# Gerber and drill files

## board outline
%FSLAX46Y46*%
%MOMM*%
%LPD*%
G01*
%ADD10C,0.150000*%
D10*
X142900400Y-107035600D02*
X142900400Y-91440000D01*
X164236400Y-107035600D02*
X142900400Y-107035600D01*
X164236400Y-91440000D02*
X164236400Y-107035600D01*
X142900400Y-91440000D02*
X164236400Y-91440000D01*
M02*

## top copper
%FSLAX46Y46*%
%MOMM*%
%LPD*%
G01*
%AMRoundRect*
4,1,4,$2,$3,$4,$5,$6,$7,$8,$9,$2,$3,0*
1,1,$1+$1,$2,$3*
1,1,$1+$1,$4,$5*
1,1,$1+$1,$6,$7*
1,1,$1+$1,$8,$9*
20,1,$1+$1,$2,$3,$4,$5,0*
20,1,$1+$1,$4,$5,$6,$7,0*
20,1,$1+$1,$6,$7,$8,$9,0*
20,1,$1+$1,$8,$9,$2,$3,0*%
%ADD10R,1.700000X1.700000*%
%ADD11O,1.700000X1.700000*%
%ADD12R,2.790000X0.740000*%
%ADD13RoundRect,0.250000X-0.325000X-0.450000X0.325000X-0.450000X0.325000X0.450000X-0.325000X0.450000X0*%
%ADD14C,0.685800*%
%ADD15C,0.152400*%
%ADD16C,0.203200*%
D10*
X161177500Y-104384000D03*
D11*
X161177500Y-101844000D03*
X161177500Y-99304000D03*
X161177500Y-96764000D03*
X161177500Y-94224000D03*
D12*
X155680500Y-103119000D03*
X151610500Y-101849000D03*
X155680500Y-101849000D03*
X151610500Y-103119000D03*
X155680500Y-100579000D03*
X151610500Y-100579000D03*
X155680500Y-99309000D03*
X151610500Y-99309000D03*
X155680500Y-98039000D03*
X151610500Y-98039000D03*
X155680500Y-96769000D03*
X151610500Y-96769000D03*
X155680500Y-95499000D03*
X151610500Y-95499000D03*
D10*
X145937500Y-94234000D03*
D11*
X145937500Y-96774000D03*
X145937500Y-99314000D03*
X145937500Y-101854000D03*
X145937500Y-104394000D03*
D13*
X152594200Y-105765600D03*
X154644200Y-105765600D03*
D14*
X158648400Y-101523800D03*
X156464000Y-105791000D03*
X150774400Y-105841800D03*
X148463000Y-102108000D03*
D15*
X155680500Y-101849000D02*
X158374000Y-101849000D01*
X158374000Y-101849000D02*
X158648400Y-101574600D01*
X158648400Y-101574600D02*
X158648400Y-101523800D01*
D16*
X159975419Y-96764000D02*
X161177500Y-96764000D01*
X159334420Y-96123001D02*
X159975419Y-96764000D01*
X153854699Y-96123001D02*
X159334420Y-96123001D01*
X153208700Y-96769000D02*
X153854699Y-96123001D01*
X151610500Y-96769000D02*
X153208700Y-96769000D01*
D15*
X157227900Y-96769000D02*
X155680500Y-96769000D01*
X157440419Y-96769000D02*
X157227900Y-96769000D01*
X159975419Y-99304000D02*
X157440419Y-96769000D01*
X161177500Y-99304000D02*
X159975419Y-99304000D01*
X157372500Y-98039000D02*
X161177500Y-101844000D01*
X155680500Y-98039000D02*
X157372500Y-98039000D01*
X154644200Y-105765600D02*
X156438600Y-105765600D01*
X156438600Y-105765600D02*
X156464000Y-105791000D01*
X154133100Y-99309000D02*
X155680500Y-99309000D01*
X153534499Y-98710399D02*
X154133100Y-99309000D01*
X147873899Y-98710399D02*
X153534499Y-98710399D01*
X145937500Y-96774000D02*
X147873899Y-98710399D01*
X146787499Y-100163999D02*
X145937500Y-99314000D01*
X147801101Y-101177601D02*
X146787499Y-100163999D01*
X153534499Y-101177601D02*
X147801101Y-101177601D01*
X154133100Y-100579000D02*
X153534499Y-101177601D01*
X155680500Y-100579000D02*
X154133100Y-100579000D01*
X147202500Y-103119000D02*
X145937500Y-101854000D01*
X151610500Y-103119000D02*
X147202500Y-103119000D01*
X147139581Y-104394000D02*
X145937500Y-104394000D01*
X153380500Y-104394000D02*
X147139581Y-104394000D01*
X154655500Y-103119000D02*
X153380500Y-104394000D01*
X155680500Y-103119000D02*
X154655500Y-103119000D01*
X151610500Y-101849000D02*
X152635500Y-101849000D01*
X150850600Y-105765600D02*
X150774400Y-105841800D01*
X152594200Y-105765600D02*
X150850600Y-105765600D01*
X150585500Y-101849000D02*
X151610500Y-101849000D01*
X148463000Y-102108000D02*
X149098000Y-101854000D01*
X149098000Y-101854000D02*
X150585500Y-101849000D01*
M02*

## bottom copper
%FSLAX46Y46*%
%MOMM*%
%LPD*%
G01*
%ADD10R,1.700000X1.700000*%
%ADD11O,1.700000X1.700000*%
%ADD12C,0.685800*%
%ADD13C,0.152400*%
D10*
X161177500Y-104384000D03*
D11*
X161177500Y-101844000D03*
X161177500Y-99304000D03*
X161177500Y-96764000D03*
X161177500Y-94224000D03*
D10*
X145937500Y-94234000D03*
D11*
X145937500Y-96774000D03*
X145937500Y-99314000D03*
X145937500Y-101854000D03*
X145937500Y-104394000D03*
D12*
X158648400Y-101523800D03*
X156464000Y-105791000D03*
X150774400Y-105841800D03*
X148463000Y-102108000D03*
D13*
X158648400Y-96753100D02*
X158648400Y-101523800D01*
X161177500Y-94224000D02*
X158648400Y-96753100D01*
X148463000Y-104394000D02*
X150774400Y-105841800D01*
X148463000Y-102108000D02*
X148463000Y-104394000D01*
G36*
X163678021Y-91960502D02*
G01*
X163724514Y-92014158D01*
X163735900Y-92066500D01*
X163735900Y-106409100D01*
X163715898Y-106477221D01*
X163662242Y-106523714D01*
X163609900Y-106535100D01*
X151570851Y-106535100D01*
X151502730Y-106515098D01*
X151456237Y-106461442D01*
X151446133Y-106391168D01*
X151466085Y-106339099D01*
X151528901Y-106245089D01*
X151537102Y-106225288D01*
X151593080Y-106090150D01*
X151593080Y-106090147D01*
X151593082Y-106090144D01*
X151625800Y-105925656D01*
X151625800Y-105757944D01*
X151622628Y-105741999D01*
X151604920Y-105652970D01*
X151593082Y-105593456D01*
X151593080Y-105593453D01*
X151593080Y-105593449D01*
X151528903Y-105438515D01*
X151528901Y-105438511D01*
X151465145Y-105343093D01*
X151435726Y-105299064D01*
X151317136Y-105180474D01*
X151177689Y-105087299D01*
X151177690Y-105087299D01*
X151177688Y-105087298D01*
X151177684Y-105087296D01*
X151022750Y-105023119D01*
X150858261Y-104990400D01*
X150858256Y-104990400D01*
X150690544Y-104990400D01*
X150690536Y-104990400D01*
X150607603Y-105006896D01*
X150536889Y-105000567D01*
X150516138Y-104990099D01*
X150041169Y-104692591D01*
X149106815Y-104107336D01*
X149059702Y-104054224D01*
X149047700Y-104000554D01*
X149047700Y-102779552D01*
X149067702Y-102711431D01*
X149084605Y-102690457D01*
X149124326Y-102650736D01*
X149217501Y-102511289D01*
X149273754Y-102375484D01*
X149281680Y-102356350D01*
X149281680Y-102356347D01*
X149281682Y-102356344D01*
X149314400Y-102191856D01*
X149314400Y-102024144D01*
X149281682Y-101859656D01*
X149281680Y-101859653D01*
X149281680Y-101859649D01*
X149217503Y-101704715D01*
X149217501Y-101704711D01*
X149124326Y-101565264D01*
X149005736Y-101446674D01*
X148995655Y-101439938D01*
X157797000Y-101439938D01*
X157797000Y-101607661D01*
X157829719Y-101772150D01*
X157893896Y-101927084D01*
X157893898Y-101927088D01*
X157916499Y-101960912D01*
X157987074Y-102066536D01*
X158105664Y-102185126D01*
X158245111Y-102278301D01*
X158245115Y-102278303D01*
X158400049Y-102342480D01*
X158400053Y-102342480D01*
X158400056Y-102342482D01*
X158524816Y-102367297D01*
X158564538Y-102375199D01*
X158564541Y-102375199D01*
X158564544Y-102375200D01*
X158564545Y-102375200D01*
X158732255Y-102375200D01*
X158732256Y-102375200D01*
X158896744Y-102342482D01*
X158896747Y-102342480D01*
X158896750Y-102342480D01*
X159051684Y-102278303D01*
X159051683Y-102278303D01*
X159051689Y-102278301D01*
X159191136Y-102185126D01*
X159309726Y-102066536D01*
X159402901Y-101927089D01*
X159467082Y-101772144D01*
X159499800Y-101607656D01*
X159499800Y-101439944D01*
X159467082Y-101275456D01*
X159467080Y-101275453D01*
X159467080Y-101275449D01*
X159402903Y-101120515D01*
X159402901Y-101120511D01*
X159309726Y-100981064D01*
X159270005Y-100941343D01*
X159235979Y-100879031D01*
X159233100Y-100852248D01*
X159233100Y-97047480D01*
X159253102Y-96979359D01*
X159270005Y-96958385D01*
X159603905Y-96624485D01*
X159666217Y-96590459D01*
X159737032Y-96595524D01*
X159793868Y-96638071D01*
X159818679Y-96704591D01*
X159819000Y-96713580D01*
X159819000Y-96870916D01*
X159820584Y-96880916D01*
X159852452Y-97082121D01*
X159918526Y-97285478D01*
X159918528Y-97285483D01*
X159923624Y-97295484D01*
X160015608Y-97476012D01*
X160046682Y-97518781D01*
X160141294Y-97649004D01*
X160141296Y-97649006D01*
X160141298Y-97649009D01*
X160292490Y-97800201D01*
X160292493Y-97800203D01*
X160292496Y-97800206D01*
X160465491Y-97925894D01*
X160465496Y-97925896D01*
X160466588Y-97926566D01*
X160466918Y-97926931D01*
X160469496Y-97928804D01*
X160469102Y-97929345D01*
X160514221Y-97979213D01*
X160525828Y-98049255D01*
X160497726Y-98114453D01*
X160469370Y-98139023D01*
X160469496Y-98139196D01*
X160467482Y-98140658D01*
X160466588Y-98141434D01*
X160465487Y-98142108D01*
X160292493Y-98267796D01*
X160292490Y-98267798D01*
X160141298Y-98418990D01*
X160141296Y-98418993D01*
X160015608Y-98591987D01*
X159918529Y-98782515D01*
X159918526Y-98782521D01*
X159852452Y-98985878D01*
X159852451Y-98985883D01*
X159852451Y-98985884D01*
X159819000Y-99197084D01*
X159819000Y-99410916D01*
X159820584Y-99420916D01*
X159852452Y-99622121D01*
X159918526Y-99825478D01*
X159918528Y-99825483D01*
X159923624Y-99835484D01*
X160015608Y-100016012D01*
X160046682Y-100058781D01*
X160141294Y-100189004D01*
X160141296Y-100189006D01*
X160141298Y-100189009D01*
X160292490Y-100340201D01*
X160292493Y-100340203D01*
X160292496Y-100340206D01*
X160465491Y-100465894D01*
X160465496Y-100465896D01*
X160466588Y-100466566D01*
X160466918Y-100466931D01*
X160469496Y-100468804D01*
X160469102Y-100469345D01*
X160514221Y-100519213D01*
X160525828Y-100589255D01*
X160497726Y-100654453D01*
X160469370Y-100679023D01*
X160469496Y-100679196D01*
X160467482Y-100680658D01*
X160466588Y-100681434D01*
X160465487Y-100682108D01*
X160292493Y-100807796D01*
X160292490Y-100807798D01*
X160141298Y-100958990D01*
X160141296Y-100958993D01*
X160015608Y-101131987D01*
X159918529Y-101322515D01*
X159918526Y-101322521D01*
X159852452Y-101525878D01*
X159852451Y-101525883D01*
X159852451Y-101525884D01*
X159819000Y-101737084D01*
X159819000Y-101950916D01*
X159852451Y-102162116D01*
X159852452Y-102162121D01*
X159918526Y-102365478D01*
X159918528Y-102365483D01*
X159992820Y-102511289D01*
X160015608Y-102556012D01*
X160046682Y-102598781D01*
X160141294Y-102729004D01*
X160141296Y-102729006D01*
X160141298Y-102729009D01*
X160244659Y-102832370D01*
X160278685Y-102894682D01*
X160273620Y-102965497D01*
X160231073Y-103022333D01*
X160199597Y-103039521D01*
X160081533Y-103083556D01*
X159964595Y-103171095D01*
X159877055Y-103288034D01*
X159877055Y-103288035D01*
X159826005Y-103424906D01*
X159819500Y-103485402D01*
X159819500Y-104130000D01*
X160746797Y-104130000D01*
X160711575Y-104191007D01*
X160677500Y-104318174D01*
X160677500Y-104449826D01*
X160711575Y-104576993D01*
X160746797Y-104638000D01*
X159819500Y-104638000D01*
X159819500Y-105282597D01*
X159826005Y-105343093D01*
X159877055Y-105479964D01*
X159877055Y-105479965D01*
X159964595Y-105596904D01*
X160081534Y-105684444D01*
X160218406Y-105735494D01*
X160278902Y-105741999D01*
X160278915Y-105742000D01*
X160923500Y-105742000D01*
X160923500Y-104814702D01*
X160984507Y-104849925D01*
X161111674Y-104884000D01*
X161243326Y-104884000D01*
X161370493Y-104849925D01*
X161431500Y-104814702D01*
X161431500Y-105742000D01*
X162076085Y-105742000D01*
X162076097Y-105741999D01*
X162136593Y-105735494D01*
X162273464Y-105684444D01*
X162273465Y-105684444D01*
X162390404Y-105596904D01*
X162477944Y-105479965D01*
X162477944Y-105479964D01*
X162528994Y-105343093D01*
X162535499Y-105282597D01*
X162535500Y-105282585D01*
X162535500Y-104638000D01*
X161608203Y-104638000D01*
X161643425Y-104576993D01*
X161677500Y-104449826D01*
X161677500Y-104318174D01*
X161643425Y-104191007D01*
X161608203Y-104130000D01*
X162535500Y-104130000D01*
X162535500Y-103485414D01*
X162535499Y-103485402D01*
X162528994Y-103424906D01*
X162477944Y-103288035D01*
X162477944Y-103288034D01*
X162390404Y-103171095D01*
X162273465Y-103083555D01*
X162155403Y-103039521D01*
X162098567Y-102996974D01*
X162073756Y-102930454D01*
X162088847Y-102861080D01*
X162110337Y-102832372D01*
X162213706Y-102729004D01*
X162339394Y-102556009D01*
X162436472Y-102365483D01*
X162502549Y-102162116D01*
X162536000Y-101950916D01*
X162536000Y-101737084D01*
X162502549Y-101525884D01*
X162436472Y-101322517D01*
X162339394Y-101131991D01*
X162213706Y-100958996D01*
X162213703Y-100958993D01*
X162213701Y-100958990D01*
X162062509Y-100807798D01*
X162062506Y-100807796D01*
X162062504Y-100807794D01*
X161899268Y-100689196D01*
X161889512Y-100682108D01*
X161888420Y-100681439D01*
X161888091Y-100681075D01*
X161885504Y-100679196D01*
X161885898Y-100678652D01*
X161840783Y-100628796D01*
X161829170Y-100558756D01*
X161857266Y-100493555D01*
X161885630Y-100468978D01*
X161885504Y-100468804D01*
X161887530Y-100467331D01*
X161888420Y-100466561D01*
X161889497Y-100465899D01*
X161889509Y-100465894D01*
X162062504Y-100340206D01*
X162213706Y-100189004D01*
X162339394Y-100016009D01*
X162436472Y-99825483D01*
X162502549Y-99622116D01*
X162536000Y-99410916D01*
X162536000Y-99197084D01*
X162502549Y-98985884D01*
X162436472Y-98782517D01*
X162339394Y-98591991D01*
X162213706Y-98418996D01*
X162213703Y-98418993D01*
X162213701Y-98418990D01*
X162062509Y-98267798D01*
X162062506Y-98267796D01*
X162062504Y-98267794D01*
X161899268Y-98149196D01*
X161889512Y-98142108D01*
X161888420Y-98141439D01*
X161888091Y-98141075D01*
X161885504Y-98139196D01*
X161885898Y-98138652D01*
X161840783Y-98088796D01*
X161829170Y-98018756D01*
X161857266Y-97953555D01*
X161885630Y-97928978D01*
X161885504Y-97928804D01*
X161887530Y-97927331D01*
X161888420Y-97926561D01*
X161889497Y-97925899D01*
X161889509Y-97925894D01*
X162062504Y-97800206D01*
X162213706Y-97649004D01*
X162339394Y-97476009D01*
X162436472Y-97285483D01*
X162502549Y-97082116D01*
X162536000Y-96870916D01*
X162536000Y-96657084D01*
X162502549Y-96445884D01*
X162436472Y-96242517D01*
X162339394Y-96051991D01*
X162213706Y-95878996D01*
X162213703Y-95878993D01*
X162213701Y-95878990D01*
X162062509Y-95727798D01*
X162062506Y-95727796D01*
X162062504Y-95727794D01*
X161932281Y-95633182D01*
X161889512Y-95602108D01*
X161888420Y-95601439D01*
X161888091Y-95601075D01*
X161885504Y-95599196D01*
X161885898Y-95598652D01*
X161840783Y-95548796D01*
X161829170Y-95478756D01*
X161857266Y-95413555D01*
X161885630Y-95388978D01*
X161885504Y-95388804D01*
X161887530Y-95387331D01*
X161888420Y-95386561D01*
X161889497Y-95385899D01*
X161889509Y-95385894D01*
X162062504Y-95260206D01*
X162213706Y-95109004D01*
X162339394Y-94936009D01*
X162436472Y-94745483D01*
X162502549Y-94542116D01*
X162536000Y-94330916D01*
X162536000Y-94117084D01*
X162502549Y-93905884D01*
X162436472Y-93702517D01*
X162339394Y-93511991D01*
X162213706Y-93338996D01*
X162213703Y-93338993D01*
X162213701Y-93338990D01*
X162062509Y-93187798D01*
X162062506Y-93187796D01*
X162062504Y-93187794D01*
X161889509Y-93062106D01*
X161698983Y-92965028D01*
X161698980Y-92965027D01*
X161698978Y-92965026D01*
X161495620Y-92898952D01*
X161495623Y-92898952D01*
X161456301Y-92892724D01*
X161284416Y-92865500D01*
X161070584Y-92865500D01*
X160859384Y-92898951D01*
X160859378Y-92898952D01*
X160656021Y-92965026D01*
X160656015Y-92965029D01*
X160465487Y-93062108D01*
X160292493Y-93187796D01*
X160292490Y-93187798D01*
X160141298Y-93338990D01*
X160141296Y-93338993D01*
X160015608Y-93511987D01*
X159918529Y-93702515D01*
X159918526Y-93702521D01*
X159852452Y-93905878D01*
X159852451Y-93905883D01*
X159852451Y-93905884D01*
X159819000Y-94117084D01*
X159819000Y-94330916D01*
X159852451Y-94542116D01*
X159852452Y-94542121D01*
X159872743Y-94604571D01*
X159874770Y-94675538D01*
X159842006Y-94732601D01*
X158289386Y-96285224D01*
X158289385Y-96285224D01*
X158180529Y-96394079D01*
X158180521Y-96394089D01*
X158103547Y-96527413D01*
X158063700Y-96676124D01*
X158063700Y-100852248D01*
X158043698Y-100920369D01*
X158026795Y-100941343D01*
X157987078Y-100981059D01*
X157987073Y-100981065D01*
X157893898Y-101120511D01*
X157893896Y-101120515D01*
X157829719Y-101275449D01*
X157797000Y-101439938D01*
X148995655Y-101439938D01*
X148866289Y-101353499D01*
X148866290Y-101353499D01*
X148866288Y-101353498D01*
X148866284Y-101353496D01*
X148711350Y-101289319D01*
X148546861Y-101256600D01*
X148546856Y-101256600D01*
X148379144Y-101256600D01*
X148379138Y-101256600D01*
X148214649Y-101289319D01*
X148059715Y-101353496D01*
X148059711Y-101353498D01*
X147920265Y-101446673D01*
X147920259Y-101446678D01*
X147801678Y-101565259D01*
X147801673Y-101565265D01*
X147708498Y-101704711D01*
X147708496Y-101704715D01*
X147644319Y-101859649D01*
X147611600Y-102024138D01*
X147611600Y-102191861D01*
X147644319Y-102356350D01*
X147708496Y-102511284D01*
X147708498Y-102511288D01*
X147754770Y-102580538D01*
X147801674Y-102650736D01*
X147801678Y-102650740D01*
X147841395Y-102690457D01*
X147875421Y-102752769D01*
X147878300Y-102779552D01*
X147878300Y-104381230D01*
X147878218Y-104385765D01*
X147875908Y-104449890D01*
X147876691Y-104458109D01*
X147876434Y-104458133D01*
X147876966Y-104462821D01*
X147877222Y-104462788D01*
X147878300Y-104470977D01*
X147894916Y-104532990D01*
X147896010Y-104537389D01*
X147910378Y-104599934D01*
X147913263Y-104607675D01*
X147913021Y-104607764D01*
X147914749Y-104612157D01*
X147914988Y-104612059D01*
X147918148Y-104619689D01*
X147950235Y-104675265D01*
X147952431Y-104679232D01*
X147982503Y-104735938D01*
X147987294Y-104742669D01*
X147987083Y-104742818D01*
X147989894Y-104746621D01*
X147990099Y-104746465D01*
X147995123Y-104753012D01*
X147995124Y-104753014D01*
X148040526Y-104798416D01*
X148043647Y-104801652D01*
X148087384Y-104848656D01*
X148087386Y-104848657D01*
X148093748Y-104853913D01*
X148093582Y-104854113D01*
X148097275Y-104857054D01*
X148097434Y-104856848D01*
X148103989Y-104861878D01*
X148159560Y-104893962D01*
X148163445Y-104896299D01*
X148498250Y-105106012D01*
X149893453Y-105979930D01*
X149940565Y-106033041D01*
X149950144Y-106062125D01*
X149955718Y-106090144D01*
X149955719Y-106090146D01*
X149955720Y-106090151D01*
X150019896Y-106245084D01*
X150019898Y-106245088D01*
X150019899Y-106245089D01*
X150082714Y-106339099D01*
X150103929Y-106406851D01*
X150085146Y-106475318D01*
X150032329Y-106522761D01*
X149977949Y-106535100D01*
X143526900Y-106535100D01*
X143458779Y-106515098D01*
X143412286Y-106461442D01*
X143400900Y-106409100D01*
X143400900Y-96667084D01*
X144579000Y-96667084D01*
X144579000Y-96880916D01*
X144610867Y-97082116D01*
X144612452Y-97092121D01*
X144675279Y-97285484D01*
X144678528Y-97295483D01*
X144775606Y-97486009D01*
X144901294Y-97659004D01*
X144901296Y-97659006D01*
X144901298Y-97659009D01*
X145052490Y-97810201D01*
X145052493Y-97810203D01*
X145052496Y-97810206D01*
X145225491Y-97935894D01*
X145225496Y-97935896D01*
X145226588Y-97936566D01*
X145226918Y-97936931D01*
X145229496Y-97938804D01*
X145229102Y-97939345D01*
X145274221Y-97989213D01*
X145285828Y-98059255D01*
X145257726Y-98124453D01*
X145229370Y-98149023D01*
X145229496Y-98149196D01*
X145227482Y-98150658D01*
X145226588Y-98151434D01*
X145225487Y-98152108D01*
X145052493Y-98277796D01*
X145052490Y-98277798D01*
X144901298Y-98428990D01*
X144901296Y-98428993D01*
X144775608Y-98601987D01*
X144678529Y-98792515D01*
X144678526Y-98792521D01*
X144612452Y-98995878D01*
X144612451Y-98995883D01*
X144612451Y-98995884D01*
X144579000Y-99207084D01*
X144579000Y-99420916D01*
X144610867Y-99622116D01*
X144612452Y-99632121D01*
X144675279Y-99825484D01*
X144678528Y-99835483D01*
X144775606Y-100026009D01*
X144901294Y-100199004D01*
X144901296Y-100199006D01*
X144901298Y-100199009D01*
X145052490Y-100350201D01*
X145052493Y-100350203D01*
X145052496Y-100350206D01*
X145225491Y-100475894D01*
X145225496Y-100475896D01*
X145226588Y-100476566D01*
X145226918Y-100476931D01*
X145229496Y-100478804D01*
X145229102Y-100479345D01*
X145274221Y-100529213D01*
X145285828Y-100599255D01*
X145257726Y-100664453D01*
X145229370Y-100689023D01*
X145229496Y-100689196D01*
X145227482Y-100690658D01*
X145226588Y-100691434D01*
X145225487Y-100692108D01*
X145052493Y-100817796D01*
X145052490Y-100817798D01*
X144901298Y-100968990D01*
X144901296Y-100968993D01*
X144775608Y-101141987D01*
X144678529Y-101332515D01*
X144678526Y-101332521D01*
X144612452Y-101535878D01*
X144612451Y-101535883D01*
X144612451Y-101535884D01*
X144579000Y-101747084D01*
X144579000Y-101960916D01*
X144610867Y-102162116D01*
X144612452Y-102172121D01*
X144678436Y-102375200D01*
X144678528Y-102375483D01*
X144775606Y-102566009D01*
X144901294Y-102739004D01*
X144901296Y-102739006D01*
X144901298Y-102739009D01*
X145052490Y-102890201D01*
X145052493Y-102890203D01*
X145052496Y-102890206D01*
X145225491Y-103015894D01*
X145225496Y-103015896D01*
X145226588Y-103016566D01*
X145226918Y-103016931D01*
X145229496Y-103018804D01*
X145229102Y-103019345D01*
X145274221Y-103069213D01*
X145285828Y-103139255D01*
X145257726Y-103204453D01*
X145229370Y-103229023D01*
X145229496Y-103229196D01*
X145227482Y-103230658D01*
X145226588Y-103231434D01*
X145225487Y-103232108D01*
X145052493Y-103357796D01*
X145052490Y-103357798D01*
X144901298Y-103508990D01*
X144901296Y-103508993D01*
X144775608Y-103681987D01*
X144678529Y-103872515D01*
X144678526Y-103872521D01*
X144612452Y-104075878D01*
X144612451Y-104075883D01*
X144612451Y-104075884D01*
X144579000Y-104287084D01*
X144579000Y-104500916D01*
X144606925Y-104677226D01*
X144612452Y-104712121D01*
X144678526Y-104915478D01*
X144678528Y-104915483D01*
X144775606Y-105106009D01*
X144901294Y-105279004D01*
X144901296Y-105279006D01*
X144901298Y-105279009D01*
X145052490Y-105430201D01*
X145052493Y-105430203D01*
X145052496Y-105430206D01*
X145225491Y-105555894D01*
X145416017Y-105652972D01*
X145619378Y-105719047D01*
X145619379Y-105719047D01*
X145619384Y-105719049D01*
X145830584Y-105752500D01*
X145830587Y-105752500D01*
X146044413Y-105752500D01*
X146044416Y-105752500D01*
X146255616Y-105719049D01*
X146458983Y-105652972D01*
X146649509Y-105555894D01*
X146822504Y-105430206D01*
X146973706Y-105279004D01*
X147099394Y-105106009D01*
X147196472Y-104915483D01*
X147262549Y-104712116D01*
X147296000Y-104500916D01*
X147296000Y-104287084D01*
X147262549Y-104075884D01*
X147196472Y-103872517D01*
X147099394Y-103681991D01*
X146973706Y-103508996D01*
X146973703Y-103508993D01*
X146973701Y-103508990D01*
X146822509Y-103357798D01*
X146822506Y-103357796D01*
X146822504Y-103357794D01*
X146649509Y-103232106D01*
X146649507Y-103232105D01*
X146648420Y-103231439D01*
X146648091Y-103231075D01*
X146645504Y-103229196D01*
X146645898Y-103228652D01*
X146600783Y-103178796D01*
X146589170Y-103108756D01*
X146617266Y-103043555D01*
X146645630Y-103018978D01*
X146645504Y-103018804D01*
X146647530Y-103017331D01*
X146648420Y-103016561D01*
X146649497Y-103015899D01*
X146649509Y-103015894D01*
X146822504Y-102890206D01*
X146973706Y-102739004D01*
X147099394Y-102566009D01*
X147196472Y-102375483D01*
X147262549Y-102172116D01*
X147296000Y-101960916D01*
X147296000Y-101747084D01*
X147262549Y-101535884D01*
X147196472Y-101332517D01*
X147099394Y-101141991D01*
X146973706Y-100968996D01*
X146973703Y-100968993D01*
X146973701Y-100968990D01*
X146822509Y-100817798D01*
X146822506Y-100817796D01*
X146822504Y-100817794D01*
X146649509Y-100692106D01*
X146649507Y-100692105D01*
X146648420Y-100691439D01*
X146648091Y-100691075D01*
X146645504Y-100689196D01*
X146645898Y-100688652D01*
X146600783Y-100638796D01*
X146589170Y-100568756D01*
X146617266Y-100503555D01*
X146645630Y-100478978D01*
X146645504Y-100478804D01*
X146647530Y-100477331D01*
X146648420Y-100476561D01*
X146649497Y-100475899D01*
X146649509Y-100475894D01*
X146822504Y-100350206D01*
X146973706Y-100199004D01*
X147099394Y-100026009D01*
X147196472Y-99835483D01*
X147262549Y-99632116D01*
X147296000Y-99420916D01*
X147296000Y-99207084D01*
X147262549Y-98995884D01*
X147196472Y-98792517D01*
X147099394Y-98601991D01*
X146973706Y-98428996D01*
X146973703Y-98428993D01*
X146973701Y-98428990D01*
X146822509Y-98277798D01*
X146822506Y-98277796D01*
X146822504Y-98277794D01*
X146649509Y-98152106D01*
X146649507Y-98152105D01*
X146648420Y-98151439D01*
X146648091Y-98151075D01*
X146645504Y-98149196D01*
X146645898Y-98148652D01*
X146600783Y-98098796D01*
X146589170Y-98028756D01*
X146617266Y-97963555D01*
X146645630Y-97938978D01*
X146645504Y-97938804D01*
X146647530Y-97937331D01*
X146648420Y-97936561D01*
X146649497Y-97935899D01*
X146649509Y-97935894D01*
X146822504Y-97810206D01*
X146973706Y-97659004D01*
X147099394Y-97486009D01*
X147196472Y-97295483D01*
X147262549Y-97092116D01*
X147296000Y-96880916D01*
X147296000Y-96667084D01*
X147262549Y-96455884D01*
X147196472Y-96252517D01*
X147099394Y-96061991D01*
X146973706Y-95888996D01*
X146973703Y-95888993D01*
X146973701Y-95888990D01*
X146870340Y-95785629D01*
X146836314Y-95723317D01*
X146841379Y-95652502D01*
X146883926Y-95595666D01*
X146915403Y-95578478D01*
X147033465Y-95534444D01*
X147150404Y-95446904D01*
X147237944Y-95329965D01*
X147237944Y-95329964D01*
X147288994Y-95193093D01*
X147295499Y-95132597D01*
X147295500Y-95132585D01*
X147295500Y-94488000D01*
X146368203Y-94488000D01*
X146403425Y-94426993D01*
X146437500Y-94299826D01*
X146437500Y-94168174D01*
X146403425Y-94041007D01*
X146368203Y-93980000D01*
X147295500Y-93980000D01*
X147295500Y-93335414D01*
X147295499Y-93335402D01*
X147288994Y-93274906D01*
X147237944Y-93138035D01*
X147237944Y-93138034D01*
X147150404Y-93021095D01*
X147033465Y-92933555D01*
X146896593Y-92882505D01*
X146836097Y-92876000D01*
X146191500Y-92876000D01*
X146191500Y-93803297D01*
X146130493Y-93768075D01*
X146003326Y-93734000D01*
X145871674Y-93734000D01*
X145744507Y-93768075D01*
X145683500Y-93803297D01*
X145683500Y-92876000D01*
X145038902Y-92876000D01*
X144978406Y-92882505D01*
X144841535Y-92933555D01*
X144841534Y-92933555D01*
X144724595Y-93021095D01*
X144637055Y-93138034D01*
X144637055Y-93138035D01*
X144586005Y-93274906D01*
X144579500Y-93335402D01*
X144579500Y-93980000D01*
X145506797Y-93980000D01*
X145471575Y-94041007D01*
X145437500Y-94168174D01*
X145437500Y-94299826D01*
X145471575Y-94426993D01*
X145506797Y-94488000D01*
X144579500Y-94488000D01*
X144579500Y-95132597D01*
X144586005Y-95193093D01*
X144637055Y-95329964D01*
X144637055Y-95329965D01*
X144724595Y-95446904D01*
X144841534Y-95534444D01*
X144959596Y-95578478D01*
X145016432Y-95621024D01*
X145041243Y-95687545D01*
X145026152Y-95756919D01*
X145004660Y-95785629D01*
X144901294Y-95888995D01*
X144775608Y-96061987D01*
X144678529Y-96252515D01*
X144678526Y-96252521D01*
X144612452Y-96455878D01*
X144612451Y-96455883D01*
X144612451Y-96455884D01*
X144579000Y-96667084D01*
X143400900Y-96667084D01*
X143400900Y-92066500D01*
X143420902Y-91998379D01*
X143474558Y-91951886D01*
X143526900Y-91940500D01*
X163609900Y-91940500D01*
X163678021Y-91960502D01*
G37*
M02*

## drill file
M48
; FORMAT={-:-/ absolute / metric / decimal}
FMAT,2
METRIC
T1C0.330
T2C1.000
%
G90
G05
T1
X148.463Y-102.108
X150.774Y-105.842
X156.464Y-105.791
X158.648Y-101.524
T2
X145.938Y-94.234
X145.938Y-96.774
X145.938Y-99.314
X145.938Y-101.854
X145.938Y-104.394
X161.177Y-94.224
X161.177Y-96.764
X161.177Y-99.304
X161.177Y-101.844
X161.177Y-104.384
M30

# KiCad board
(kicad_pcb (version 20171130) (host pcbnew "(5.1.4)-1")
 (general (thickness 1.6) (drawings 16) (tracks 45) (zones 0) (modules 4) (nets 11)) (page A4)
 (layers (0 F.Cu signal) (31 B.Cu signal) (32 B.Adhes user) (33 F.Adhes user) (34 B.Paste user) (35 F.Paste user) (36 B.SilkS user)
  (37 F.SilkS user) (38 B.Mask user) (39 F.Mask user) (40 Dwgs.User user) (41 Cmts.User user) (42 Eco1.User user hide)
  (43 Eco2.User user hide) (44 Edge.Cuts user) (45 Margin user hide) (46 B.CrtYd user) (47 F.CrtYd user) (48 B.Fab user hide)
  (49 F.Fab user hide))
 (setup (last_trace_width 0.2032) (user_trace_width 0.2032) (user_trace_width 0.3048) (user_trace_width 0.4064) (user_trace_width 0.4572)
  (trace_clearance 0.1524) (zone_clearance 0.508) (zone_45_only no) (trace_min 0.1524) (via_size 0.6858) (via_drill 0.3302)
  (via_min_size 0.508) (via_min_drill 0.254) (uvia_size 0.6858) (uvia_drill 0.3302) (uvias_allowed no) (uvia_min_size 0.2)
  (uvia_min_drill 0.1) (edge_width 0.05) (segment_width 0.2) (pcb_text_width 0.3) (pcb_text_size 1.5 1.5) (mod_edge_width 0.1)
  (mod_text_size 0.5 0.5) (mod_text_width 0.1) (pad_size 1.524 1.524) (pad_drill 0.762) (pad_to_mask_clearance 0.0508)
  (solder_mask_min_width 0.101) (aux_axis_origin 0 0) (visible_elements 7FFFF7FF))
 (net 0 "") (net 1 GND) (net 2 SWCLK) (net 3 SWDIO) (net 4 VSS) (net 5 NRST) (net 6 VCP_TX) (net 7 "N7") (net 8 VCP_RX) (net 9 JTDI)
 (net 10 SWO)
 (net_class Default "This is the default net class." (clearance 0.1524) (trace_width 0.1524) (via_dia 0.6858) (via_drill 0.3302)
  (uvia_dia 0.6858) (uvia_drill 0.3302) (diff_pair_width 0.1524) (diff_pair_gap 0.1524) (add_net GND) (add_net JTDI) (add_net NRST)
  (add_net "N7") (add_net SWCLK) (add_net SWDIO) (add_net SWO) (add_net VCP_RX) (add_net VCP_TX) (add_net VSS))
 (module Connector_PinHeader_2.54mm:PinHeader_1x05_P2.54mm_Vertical (layer F.Cu) (at 161.1775 104.384 180)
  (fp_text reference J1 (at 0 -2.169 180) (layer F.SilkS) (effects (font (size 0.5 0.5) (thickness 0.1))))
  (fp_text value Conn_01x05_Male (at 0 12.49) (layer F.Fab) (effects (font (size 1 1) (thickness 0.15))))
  (pad 1 thru_hole rect (at 0 0 180) (size 1.7 1.7) (drill 1) (layers *.Cu *.Mask) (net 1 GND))
  (pad 2 thru_hole oval (at 0 2.54 180) (size 1.7 1.7) (drill 1) (layers *.Cu *.Mask) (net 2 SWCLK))
  (pad 3 thru_hole oval (at 0 5.08 180) (size 1.7 1.7) (drill 1) (layers *.Cu *.Mask) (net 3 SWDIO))
  (pad 4 thru_hole oval (at 0 7.62 180) (size 1.7 1.7) (drill 1) (layers *.Cu *.Mask) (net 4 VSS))
  (pad 5 thru_hole oval (at 0 10.16 180) (size 1.7 1.7) (drill 1) (layers *.Cu *.Mask) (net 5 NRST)))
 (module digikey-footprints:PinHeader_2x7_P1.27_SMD (layer F.Cu) (at 153.6455 99.309 270)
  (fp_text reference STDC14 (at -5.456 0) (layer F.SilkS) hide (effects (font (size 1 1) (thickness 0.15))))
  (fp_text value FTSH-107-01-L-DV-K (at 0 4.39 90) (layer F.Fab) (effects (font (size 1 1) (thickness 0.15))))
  (pad 14 smd rect (at 3.81 -2.035 270) (size 0.74 2.79) (layers F.Cu F.Paste F.Mask) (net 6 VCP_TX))
  (pad 11 smd rect (at 2.54 2.035 270) (size 0.74 2.79) (layers F.Cu F.Paste F.Mask) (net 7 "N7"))
  (pad 12 smd rect (at 2.54 -2.035 270) (size 0.74 2.79) (layers F.Cu F.Paste F.Mask) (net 5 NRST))
  (pad 13 smd rect (at 3.81 2.035 270) (size 0.74 2.79) (layers F.Cu F.Paste F.Mask) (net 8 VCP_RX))
  (pad 10 smd rect (at 1.27 -2.035 270) (size 0.74 2.79) (layers F.Cu F.Paste F.Mask) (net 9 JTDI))
  (pad 9 smd rect (at 1.27 2.035 270) (size 0.74 2.79) (layers F.Cu F.Paste F.Mask))
  (pad 8 smd rect (at 0 -2.035 270) (size 0.74 2.79) (layers F.Cu F.Paste F.Mask) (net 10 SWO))
  (pad 7 smd rect (at 0 2.035 270) (size 0.74 2.79) (layers F.Cu F.Paste F.Mask) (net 1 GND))
  (pad 6 smd rect (at -1.27 -2.035 270) (size 0.74 2.79) (layers F.Cu F.Paste F.Mask) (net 2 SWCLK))
  (pad 5 smd rect (at -1.27 2.035 270) (size 0.74 2.79) (layers F.Cu F.Paste F.Mask) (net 1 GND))
  (pad 4 smd rect (at -2.54 -2.035 270) (size 0.74 2.79) (layers F.Cu F.Paste F.Mask) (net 3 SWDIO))
  (pad 3 smd rect (at -2.54 2.035 270) (size 0.74 2.79) (layers F.Cu F.Paste F.Mask) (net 4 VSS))
  (pad 2 smd rect (at -3.81 -2.035 270) (size 0.74 2.79) (layers F.Cu F.Paste F.Mask))
  (pad 1 smd rect (at -3.81 2.035 270) (size 0.74 2.79) (layers F.Cu F.Paste F.Mask)))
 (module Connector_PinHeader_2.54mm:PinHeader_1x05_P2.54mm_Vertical (layer F.Cu) (at 145.9375 94.234)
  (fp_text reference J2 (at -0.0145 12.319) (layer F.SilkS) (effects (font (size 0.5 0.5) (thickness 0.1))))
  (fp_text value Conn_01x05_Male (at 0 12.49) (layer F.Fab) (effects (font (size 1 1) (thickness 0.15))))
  (pad 1 thru_hole rect (at 0 0) (size 1.7 1.7) (drill 1) (layers *.Cu *.Mask) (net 1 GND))
  (pad 2 thru_hole oval (at 0 2.54) (size 1.7 1.7) (drill 1) (layers *.Cu *.Mask) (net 10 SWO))
  (pad 3 thru_hole oval (at 0 5.08) (size 1.7 1.7) (drill 1) (layers *.Cu *.Mask) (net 9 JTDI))
  (pad 4 thru_hole oval (at 0 7.62) (size 1.7 1.7) (drill 1) (layers *.Cu *.Mask) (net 8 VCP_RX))
  (pad 5 thru_hole oval (at 0 10.16) (size 1.7 1.7) (drill 1) (layers *.Cu *.Mask) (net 6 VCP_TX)))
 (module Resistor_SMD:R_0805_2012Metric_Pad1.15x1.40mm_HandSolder (layer F.Cu) (at 153.6192 105.7656)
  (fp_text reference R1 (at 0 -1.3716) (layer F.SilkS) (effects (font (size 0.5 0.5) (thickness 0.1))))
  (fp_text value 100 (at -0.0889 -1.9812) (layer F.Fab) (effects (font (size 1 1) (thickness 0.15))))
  (pad 1 smd roundrect (at -1.025 0) (size 1.15 1.4) (layers F.Cu F.Paste F.Mask) (roundrect_rratio 0.217391) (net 7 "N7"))
  (pad 2 smd roundrect (at 1.025 0) (size 1.15 1.4) (layers F.Cu F.Paste F.Mask) (roundrect_rratio 0.217391) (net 1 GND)))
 (gr_line (start 142.9004 107.0356) (end 142.9004 91.44) (layer Edge.Cuts) (width 0.15))
 (gr_line (start 164.2364 107.0356) (end 142.9004 107.0356) (layer Edge.Cuts) (width 0.15))
 (gr_line (start 164.2364 91.44) (end 164.2364 107.0356) (layer Edge.Cuts) (width 0.15))
 (gr_line (start 142.9004 91.44) (end 164.2364 91.44) (layer Edge.Cuts) (width 0.15))
 (segment (start 155.6805 101.849) (end 158.374 101.849) (width 0.1524) (layer F.Cu) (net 5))
 (via (at 158.6484 101.5238) (size 0.6858) (drill 0.3302) (layers F.Cu B.Cu) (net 5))
 (segment (start 158.374 101.849) (end 158.6484 101.5746) (width 0.1524) (layer F.Cu) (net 5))
 (segment (start 158.6484 101.5746) (end 158.6484 101.5238) (width 0.1524) (layer F.Cu) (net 5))
 (segment (start 158.6484 96.7531) (end 158.6484 101.5238) (width 0.1524) (layer B.Cu) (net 5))
 (segment (start 161.1775 94.224) (end 158.6484 96.7531) (width 0.1524) (layer B.Cu) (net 5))
 (segment (start 159.975419 96.764) (end 161.1775 96.764) (width 0.2032) (layer F.Cu) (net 4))
 (segment (start 159.33442 96.123001) (end 159.975419 96.764) (width 0.2032) (layer F.Cu) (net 4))
 (segment (start 153.854699 96.123001) (end 159.33442 96.123001) (width 0.2032) (layer F.Cu) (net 4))
 (segment (start 153.2087 96.769) (end 153.854699 96.123001) (width 0.2032) (layer F.Cu) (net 4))
 (segment (start 151.6105 96.769) (end 153.2087 96.769) (width 0.2032) (layer F.Cu) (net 4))
 (segment (start 157.2279 96.769) (end 155.6805 96.769) (width 0.1524) (layer F.Cu) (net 3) (status 20))
 (segment (start 157.440419 96.769) (end 157.2279 96.769) (width 0.1524) (layer F.Cu) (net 3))
 (segment (start 159.975419 99.304) (end 157.440419 96.769) (width 0.1524) (layer F.Cu) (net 3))
 (segment (start 161.1775 99.304) (end 159.975419 99.304) (width 0.1524) (layer F.Cu) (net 3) (status 10))
 (segment (start 157.3725 98.039) (end 161.1775 101.844) (width 0.1524) (layer F.Cu) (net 2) (status 20))
 (segment (start 155.6805 98.039) (end 157.3725 98.039) (width 0.1524) (layer F.Cu) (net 2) (status 10))
 (via (at 156.464 105.791) (size 0.6858) (drill 0.3302) (layers F.Cu B.Cu) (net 1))
 (segment (start 154.6442 105.7656) (end 156.4386 105.7656) (width 0.1524) (layer F.Cu) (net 1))
 (segment (start 156.4386 105.7656) (end 156.464 105.791) (width 0.1524) (layer F.Cu) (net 1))
 (segment (start 154.1331 99.309) (end 155.6805 99.309) (width 0.1524) (layer F.Cu) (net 10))
 (segment (start 153.534499 98.710399) (end 154.1331 99.309) (width 0.1524) (layer F.Cu) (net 10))
 (segment (start 147.873899 98.710399) (end 153.534499 98.710399) (width 0.1524) (layer F.Cu) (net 10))
 (segment (start 145.9375 96.774) (end 147.873899 98.710399) (width 0.1524) (layer F.Cu) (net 10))
 (segment (start 146.787499 100.163999) (end 145.9375 99.314) (width 0.1524) (layer F.Cu) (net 9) (status 20))
 (segment (start 147.801101 101.177601) (end 146.787499 100.163999) (width 0.1524) (layer F.Cu) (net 9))
 (segment (start 153.534499 101.177601) (end 147.801101 101.177601) (width 0.1524) (layer F.Cu) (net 9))
 (segment (start 154.1331 100.579) (end 153.534499 101.177601) (width 0.1524) (layer F.Cu) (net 9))
 (segment (start 155.6805 100.579) (end 154.1331 100.579) (width 0.1524) (layer F.Cu) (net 9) (status 10))
 (segment (start 147.2025 103.119) (end 145.9375 101.854) (width 0.1524) (layer F.Cu) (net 8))
 (segment (start 151.6105 103.119) (end 147.2025 103.119) (width 0.1524) (layer F.Cu) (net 8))
 (segment (start 147.139581 104.394) (end 145.9375 104.394) (width 0.1524) (layer F.Cu) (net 6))
 (segment (start 153.3805 104.394) (end 147.139581 104.394) (width 0.1524) (layer F.Cu) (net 6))
 (segment (start 154.6555 103.119) (end 153.3805 104.394) (width 0.1524) (layer F.Cu) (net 6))
 (segment (start 155.6805 103.119) (end 154.6555 103.119) (width 0.1524) (layer F.Cu) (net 6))
 (segment (start 151.6105 101.849) (end 152.6355 101.849) (width 0.1524) (layer F.Cu) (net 7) (status 30))
 (via (at 150.7744 105.8418) (size 0.6858) (drill 0.3302) (layers F.Cu B.Cu) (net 7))
 (segment (start 150.8506 105.7656) (end 150.7744 105.8418) (width 0.1524) (layer F.Cu) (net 7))
 (segment (start 152.5942 105.7656) (end 150.8506 105.7656) (width 0.1524) (layer F.Cu) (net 7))
 (via (at 148.463 102.108) (size 0.6858) (drill 0.3302) (layers F.Cu B.Cu) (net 7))
 (segment (start 150.5855 101.849) (end 151.6105 101.849) (width 0.1524) (layer F.Cu) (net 7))
 (segment (start 148.463 102.108) (end 149.098 101.854) (width 0.1524) (layer F.Cu) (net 7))
 (segment (start 149.098 101.854) (end 150.5855 101.849) (width 0.1524) (layer F.Cu) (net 7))
 (segment (start 148.463 104.394) (end 150.7744 105.8418) (width 0.1524) (layer B.Cu) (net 7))
 (segment (start 148.463 102.108) (end 148.463 104.394) (width 0.1524) (layer B.Cu) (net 7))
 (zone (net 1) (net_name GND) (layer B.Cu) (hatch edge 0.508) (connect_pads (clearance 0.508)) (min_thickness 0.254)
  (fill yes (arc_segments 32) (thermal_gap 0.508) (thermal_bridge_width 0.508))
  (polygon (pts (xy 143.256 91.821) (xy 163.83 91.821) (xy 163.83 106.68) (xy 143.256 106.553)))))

